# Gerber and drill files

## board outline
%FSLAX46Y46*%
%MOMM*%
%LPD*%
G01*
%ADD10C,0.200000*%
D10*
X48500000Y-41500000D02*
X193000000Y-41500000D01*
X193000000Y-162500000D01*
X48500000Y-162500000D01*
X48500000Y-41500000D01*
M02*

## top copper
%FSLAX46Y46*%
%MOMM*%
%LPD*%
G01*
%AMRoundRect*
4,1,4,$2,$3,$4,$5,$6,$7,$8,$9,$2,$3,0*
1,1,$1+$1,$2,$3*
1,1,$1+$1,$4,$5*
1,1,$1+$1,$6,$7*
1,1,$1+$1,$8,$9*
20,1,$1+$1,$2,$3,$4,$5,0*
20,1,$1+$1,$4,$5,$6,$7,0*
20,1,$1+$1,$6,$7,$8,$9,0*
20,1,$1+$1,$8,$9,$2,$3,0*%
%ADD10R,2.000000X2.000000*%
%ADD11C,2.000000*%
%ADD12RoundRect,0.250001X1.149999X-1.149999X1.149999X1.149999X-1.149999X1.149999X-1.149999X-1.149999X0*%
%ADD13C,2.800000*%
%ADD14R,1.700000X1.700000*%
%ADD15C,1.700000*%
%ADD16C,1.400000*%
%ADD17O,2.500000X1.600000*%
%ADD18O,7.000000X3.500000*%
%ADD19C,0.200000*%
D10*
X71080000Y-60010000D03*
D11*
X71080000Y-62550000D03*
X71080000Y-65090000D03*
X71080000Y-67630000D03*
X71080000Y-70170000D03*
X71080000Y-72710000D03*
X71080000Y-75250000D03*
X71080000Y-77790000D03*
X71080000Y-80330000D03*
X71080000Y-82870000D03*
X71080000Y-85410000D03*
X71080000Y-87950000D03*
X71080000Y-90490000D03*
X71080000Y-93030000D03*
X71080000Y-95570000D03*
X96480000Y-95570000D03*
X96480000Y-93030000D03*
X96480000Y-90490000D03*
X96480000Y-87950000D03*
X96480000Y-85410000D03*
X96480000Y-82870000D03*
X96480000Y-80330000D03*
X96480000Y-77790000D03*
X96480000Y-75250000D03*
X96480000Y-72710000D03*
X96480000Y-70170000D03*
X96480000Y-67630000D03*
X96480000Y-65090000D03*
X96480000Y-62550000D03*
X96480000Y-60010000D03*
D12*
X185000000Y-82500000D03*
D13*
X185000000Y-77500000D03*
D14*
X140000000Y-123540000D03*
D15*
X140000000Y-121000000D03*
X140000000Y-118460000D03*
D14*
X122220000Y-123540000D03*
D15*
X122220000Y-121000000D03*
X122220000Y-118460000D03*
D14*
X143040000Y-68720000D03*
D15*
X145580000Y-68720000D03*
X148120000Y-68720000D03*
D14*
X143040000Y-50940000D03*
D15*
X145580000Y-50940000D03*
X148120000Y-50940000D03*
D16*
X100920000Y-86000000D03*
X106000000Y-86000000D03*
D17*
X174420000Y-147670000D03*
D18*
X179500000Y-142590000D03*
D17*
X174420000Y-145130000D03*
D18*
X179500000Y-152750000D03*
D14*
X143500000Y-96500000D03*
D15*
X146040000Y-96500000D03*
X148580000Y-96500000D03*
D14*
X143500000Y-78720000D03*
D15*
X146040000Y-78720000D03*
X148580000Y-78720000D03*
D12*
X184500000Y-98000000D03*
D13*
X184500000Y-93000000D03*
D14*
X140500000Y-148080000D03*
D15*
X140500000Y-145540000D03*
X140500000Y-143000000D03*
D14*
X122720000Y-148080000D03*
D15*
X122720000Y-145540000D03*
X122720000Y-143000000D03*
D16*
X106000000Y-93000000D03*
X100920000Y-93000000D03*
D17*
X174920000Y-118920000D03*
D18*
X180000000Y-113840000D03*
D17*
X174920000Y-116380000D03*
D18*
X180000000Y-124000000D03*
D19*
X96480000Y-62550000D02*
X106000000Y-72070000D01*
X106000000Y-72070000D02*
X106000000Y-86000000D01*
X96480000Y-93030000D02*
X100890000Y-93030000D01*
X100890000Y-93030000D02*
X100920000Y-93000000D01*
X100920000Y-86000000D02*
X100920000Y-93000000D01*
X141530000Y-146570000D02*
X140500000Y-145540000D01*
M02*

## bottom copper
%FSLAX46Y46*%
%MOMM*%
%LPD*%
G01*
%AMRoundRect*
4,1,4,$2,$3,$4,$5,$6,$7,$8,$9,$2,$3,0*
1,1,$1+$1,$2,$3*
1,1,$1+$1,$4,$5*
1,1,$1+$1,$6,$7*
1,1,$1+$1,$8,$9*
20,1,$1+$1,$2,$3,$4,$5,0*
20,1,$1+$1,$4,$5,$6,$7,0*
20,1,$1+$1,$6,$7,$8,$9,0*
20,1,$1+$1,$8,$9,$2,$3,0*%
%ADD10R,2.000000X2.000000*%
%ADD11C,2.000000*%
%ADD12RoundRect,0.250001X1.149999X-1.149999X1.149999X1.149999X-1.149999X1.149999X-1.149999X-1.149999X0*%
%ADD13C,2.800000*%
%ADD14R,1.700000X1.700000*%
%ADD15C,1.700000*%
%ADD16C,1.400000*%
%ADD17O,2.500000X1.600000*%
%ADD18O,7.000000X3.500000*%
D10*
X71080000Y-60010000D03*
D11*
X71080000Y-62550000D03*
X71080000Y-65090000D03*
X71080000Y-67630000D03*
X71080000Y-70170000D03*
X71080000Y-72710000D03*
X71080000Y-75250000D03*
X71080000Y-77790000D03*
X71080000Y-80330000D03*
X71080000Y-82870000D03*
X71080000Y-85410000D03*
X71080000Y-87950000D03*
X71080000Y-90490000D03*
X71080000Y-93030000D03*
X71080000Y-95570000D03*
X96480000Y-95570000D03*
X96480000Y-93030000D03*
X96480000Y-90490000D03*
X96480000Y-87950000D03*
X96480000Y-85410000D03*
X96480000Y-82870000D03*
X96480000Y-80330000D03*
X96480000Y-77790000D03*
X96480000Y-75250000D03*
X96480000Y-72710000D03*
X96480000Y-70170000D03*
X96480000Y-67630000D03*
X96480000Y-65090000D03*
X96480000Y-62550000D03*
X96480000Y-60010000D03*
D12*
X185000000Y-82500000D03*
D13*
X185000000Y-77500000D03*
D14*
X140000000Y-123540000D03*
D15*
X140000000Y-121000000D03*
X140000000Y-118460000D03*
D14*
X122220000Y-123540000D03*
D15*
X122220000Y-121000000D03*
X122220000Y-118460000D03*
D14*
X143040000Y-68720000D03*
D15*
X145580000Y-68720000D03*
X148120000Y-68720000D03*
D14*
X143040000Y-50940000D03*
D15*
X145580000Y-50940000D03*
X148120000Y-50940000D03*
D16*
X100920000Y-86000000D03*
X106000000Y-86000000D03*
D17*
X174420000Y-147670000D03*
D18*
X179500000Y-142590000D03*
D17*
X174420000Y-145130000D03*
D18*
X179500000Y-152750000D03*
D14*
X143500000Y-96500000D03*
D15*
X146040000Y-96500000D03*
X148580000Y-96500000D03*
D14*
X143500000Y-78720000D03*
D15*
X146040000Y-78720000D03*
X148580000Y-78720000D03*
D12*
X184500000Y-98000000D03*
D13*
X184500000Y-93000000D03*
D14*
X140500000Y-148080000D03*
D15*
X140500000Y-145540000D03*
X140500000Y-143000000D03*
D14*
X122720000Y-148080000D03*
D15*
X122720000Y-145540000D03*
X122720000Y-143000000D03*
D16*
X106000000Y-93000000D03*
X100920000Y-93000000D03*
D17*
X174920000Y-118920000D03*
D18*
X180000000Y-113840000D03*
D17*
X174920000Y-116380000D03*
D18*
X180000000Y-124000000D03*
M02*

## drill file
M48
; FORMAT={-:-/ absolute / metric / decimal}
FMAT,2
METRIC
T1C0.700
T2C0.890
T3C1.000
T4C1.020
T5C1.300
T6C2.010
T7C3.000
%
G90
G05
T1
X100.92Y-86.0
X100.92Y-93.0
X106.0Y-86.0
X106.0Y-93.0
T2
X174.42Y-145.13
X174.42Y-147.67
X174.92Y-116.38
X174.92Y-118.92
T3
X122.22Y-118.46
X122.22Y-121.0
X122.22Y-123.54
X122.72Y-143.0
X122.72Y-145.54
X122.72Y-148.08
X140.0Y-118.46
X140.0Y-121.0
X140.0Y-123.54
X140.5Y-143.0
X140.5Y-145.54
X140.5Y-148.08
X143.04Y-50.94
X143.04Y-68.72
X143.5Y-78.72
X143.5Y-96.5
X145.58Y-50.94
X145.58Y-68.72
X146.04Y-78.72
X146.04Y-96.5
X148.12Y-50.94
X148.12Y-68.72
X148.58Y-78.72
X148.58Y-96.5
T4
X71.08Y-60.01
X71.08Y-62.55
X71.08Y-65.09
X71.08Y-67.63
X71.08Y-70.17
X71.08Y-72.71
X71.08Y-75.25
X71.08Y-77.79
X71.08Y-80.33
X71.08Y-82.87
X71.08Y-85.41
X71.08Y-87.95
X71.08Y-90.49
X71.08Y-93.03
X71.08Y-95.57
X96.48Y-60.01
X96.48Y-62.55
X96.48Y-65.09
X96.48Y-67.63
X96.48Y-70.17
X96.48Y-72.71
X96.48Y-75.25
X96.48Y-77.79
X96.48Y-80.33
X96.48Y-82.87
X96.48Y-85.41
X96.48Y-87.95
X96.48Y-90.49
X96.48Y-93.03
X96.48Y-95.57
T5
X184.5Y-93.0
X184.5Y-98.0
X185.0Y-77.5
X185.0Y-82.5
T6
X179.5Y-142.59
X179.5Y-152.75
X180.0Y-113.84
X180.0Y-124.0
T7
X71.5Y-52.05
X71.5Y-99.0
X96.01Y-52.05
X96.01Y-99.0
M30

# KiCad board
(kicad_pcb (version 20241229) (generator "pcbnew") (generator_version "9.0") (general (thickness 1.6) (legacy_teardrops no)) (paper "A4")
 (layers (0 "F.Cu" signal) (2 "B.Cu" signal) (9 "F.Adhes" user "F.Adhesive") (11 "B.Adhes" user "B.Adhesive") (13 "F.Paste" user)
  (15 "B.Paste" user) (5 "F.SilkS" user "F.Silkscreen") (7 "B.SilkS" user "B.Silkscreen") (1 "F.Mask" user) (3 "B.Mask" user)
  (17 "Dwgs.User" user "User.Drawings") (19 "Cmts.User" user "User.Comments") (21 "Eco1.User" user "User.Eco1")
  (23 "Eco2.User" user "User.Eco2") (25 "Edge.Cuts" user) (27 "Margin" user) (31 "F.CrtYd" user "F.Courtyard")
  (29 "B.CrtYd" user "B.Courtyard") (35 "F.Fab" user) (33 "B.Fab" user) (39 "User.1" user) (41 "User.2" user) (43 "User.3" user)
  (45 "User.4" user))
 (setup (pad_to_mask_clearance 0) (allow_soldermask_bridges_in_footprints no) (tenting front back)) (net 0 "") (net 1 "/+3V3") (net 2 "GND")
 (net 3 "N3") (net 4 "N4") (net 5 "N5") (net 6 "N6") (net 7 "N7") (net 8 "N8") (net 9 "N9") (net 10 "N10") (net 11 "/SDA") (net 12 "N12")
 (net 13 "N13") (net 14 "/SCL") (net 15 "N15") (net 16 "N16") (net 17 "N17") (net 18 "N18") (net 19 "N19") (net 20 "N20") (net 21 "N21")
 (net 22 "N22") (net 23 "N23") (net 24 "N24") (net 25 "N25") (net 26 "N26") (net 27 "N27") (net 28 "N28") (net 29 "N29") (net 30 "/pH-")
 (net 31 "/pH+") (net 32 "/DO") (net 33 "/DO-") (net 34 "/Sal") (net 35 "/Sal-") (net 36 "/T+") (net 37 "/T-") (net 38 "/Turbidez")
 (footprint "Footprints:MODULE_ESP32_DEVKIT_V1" (layer "F.Cu") (at 83.78 75.525)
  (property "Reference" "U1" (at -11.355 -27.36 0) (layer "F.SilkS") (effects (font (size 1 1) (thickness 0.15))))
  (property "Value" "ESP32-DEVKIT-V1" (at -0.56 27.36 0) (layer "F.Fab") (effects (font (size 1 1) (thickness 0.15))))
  (pad "" np_thru_hole circle (at -12.28 -23.475) (size 3 3) (drill 3) (layers "*.Cu" "*.Mask"))
  (pad "" np_thru_hole circle (at -12.28 23.475) (size 3 3) (drill 3) (layers "*.Cu" "*.Mask"))
  (pad "" np_thru_hole circle (at 12.23 -23.475) (size 3 3) (drill 3) (layers "*.Cu" "*.Mask"))
  (pad "" np_thru_hole circle (at 12.23 23.475) (size 3 3) (drill 3) (layers "*.Cu" "*.Mask"))
  (pad "1" thru_hole rect (at -12.7 -15.515) (size 2 2) (drill 1.02) (layers "*.Cu" "*.Mask") (remove_unused_layers no) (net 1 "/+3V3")
   (solder_mask_margin 0.102))
  (pad "2" thru_hole circle (at -12.7 -12.975) (size 2 2) (drill 1.02) (layers "*.Cu" "*.Mask") (remove_unused_layers no) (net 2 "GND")
   (solder_mask_margin 0.102))
  (pad "3" thru_hole circle (at -12.7 -10.435) (size 2 2) (drill 1.02) (layers "*.Cu" "*.Mask") (remove_unused_layers no) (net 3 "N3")
   (solder_mask_margin 0.102))
  (pad "4" thru_hole circle (at -12.7 -7.895) (size 2 2) (drill 1.02) (layers "*.Cu" "*.Mask") (remove_unused_layers no) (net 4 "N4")
   (solder_mask_margin 0.102))
  (pad "5" thru_hole circle (at -12.7 -5.355) (size 2 2) (drill 1.02) (layers "*.Cu" "*.Mask") (remove_unused_layers no) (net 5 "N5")
   (solder_mask_margin 0.102))
  (pad "6" thru_hole circle (at -12.7 -2.815) (size 2 2) (drill 1.02) (layers "*.Cu" "*.Mask") (remove_unused_layers no) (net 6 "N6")
   (solder_mask_margin 0.102))
  (pad "7" thru_hole circle (at -12.7 -0.275) (size 2 2) (drill 1.02) (layers "*.Cu" "*.Mask") (remove_unused_layers no) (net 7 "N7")
   (solder_mask_margin 0.102))
  (pad "8" thru_hole circle (at -12.7 2.265) (size 2 2) (drill 1.02) (layers "*.Cu" "*.Mask") (remove_unused_layers no) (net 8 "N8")
   (solder_mask_margin 0.102))
  (pad "9" thru_hole circle (at -12.7 4.805) (size 2 2) (drill 1.02) (layers "*.Cu" "*.Mask") (remove_unused_layers no) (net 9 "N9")
   (solder_mask_margin 0.102))
  (pad "10" thru_hole circle (at -12.7 7.345) (size 2 2) (drill 1.02) (layers "*.Cu" "*.Mask") (remove_unused_layers no) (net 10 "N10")
   (solder_mask_margin 0.102))
  (pad "11" thru_hole circle (at -12.7 9.885) (size 2 2) (drill 1.02) (layers "*.Cu" "*.Mask") (remove_unused_layers no) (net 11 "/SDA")
   (solder_mask_margin 0.102))
  (pad "12" thru_hole circle (at -12.7 12.425) (size 2 2) (drill 1.02) (layers "*.Cu" "*.Mask") (remove_unused_layers no) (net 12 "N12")
   (solder_mask_margin 0.102))
  (pad "13" thru_hole circle (at -12.7 14.965) (size 2 2) (drill 1.02) (layers "*.Cu" "*.Mask") (remove_unused_layers no) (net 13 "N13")
   (solder_mask_margin 0.102))
  (pad "14" thru_hole circle (at -12.7 17.505) (size 2 2) (drill 1.02) (layers "*.Cu" "*.Mask") (remove_unused_layers no) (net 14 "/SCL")
   (solder_mask_margin 0.102))
  (pad "15" thru_hole circle (at -12.7 20.045) (size 2 2) (drill 1.02) (layers "*.Cu" "*.Mask") (remove_unused_layers no) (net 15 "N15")
   (solder_mask_margin 0.102))
  (pad "16" thru_hole circle (at 12.7 20.045) (size 2 2) (drill 1.02) (layers "*.Cu" "*.Mask") (remove_unused_layers no) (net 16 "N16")
   (solder_mask_margin 0.102))
  (pad "17" thru_hole circle (at 12.7 17.505) (size 2 2) (drill 1.02) (layers "*.Cu" "*.Mask") (remove_unused_layers no) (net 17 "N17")
   (solder_mask_margin 0.102))
  (pad "18" thru_hole circle (at 12.7 14.965) (size 2 2) (drill 1.02) (layers "*.Cu" "*.Mask") (remove_unused_layers no) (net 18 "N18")
   (solder_mask_margin 0.102))
  (pad "19" thru_hole circle (at 12.7 12.425) (size 2 2) (drill 1.02) (layers "*.Cu" "*.Mask") (remove_unused_layers no) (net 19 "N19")
   (solder_mask_margin 0.102))
  (pad "20" thru_hole circle (at 12.7 9.885) (size 2 2) (drill 1.02) (layers "*.Cu" "*.Mask") (remove_unused_layers no) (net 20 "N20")
   (solder_mask_margin 0.102))
  (pad "21" thru_hole circle (at 12.7 7.345) (size 2 2) (drill 1.02) (layers "*.Cu" "*.Mask") (remove_unused_layers no) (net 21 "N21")
   (solder_mask_margin 0.102))
  (pad "22" thru_hole circle (at 12.7 4.805) (size 2 2) (drill 1.02) (layers "*.Cu" "*.Mask") (remove_unused_layers no) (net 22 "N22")
   (solder_mask_margin 0.102))
  (pad "23" thru_hole circle (at 12.7 2.265) (size 2 2) (drill 1.02) (layers "*.Cu" "*.Mask") (remove_unused_layers no) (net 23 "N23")
   (solder_mask_margin 0.102))
  (pad "24" thru_hole circle (at 12.7 -0.275) (size 2 2) (drill 1.02) (layers "*.Cu" "*.Mask") (remove_unused_layers no) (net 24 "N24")
   (solder_mask_margin 0.102))
  (pad "25" thru_hole circle (at 12.7 -2.815) (size 2 2) (drill 1.02) (layers "*.Cu" "*.Mask") (remove_unused_layers no) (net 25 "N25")
   (solder_mask_margin 0.102))
  (pad "26" thru_hole circle (at 12.7 -5.355) (size 2 2) (drill 1.02) (layers "*.Cu" "*.Mask") (remove_unused_layers no) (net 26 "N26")
   (solder_mask_margin 0.102))
  (pad "27" thru_hole circle (at 12.7 -7.895) (size 2 2) (drill 1.02) (layers "*.Cu" "*.Mask") (remove_unused_layers no) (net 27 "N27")
   (solder_mask_margin 0.102))
  (pad "28" thru_hole circle (at 12.7 -10.435) (size 2 2) (drill 1.02) (layers "*.Cu" "*.Mask") (remove_unused_layers no) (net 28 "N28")
   (solder_mask_margin 0.102))
  (pad "29" thru_hole circle (at 12.7 -12.975) (size 2 2) (drill 1.02) (layers "*.Cu" "*.Mask") (remove_unused_layers no) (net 2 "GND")
   (solder_mask_margin 0.102))
  (pad "30" thru_hole circle (at 12.7 -15.515) (size 2 2) (drill 1.02) (layers "*.Cu" "*.Mask") (remove_unused_layers no) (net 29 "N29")
   (solder_mask_margin 0.102))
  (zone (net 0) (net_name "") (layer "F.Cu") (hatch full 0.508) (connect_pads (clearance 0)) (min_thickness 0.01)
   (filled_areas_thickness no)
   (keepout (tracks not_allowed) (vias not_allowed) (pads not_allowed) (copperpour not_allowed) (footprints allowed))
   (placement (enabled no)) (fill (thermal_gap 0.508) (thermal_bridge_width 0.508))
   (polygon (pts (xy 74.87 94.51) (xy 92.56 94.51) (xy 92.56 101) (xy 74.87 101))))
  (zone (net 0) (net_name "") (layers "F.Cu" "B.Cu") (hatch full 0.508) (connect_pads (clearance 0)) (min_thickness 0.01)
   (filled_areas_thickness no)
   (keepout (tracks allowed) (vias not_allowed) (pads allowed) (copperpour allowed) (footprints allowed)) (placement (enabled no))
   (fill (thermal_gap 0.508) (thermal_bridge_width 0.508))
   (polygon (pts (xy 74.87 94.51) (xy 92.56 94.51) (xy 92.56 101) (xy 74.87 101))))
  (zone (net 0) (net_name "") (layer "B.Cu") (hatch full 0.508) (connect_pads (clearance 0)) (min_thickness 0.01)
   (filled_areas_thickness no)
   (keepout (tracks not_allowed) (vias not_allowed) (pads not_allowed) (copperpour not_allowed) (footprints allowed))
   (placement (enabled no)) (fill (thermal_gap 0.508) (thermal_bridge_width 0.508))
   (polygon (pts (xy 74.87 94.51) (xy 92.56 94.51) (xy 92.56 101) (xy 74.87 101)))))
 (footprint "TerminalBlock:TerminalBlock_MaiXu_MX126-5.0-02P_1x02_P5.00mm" (layer "F.Cu") (at 185 82.5 90)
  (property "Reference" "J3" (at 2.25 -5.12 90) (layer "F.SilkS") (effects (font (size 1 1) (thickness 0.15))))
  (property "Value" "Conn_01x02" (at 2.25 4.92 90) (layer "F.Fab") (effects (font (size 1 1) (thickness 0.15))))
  (pad "1" thru_hole roundrect (at 0 0 90) (size 2.8 2.8) (drill 1.3) (layers "*.Cu" "*.Mask") (remove_unused_layers no)
   (roundrect_rratio 0.089286) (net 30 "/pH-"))
  (pad "2" thru_hole circle (at 5 0 90) (size 2.8 2.8) (drill 1.3) (layers "*.Cu" "*.Mask") (remove_unused_layers no) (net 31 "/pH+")))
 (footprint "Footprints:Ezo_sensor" (layer "F.Cu") (at 119 114.46 90)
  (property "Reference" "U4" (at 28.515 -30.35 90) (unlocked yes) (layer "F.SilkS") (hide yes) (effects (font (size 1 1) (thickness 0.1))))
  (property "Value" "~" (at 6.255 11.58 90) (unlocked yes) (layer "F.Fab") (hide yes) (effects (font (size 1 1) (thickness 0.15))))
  (pad "1" thru_hole rect (at -9.08 21 180) (size 1.7 1.7) (drill 1) (layers "*.Cu" "*.Mask") (remove_unused_layers no) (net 1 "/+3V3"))
  (pad "2" thru_hole circle (at -6.54 21 180) (size 1.7 1.7) (drill 1) (layers "*.Cu" "*.Mask") (remove_unused_layers no) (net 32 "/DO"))
  (pad "3" thru_hole circle (at -4 21 180) (size 1.7 1.7) (drill 1) (layers "*.Cu" "*.Mask") (remove_unused_layers no) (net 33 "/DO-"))
  (pad "4" thru_hole rect (at -9.08 3.22 180) (size 1.7 1.7) (drill 1) (layers "*.Cu" "*.Mask") (remove_unused_layers no) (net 2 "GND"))
  (pad "5" thru_hole circle (at -6.54 3.22 180) (size 1.7 1.7) (drill 1) (layers "*.Cu" "*.Mask") (remove_unused_layers no) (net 11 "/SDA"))
  (pad "6" thru_hole circle (at -4 3.22 180) (size 1.7 1.7) (drill 1) (layers "*.Cu" "*.Mask") (remove_unused_layers no) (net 14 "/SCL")))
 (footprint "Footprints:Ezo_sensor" (layer "F.Cu") (at 112.875 90.8)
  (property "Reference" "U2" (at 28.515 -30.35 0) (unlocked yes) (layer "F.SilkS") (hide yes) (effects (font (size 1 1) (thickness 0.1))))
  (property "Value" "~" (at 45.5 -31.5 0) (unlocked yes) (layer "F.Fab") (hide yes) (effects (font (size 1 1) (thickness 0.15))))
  (pad "1" thru_hole rect (at 30.165 -22.08 90) (size 1.7 1.7) (drill 1) (layers "*.Cu" "*.Mask") (remove_unused_layers no) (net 1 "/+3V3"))
  (pad "2" thru_hole circle (at 32.705 -22.08 90) (size 1.7 1.7) (drill 1) (layers "*.Cu" "*.Mask") (remove_unused_layers no)
   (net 31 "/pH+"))
  (pad "3" thru_hole circle (at 35.245 -22.08 90) (size 1.7 1.7) (drill 1) (layers "*.Cu" "*.Mask") (remove_unused_layers no)
   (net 30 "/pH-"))
  (pad "4" thru_hole rect (at 30.165 -39.86 90) (size 1.7 1.7) (drill 1) (layers "*.Cu" "*.Mask") (remove_unused_layers no) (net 2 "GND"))
  (pad "5" thru_hole circle (at 32.705 -39.86 90) (size 1.7 1.7) (drill 1) (layers "*.Cu" "*.Mask") (remove_unused_layers no)
   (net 11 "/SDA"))
  (pad "6" thru_hole circle (at 35.245 -39.86 90) (size 1.7 1.7) (drill 1) (layers "*.Cu" "*.Mask") (remove_unused_layers no)
   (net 14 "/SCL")))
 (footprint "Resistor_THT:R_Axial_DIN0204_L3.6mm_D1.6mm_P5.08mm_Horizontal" (layer "F.Cu") (at 100.92 86)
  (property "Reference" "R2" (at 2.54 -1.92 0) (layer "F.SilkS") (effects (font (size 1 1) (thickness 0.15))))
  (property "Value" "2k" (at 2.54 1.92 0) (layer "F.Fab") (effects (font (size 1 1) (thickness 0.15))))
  (pad "1" thru_hole circle (at 0 0) (size 1.4 1.4) (drill 0.7) (layers "*.Cu" "*.Mask") (remove_unused_layers no) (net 17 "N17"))
  (pad "2" thru_hole circle (at 5.08 0) (size 1.4 1.4) (drill 0.7) (layers "*.Cu" "*.Mask") (remove_unused_layers no) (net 2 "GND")))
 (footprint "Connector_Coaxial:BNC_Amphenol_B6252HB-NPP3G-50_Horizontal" (layer "F.Cu") (at 174.42 147.67 -90)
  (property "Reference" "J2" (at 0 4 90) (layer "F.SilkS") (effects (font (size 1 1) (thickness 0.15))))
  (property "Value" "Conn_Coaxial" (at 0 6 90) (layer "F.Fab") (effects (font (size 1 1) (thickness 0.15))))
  (pad "1" thru_hole oval (at 0 0 270) (size 1.6 2.5) (drill 0.89) (layers "*.Cu" "*.Mask") (remove_unused_layers no) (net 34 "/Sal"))
  (pad "2" thru_hole oval (at -5.08 -5.08 270) (size 3.5 7) (drill 2.01) (layers "*.Cu" "*.Mask") (remove_unused_layers no) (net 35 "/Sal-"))
  (pad "2" thru_hole oval (at -2.54 0 270) (size 1.6 2.5) (drill 0.89) (layers "*.Cu" "*.Mask") (remove_unused_layers no) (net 35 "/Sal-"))
  (pad "2" thru_hole oval (at 5.08 -5.08 270) (size 3.5 7) (drill 2.01) (layers "*.Cu" "*.Mask") (remove_unused_layers no) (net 35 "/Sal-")))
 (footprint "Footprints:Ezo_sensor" (layer "F.Cu") (at 113.335 118.58)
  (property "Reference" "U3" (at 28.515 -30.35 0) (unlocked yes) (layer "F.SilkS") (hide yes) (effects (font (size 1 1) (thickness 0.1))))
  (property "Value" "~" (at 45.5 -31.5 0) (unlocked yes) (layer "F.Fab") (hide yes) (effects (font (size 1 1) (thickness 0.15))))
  (pad "1" thru_hole rect (at 30.165 -22.08 90) (size 1.7 1.7) (drill 1) (layers "*.Cu" "*.Mask") (remove_unused_layers no) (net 1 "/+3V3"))
  (pad "2" thru_hole circle (at 32.705 -22.08 90) (size 1.7 1.7) (drill 1) (layers "*.Cu" "*.Mask") (remove_unused_layers no) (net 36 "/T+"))
  (pad "3" thru_hole circle (at 35.245 -22.08 90) (size 1.7 1.7) (drill 1) (layers "*.Cu" "*.Mask") (remove_unused_layers no) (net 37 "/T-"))
  (pad "4" thru_hole rect (at 30.165 -39.86 90) (size 1.7 1.7) (drill 1) (layers "*.Cu" "*.Mask") (remove_unused_layers no) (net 2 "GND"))
  (pad "5" thru_hole circle (at 32.705 -39.86 90) (size 1.7 1.7) (drill 1) (layers "*.Cu" "*.Mask") (remove_unused_layers no)
   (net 11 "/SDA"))
  (pad "6" thru_hole circle (at 35.245 -39.86 90) (size 1.7 1.7) (drill 1) (layers "*.Cu" "*.Mask") (remove_unused_layers no)
   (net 14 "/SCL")))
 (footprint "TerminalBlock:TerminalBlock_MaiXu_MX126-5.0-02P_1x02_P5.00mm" (layer "F.Cu") (at 184.5 98 90)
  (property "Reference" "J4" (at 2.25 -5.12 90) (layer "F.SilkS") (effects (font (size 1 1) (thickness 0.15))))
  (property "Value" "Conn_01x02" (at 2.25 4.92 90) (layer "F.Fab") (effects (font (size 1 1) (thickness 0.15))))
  (pad "1" thru_hole roundrect (at 0 0 90) (size 2.8 2.8) (drill 1.3) (layers "*.Cu" "*.Mask") (remove_unused_layers no)
   (roundrect_rratio 0.089286) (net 37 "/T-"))
  (pad "2" thru_hole circle (at 5 0 90) (size 2.8 2.8) (drill 1.3) (layers "*.Cu" "*.Mask") (remove_unused_layers no) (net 36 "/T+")))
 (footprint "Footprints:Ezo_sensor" (layer "F.Cu") (at 119.5 139 90)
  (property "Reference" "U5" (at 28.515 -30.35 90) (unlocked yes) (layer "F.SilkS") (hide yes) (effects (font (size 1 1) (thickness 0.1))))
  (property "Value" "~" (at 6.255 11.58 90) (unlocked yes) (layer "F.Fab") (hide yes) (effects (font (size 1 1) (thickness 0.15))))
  (pad "1" thru_hole rect (at -9.08 21 180) (size 1.7 1.7) (drill 1) (layers "*.Cu" "*.Mask") (remove_unused_layers no) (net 1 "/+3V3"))
  (pad "2" thru_hole circle (at -6.54 21 180) (size 1.7 1.7) (drill 1) (layers "*.Cu" "*.Mask") (remove_unused_layers no) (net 34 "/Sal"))
  (pad "3" thru_hole circle (at -4 21 180) (size 1.7 1.7) (drill 1) (layers "*.Cu" "*.Mask") (remove_unused_layers no) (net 35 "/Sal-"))
  (pad "4" thru_hole rect (at -9.08 3.22 180) (size 1.7 1.7) (drill 1) (layers "*.Cu" "*.Mask") (remove_unused_layers no) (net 2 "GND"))
  (pad "5" thru_hole circle (at -6.54 3.22 180) (size 1.7 1.7) (drill 1) (layers "*.Cu" "*.Mask") (remove_unused_layers no) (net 11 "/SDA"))
  (pad "6" thru_hole circle (at -4 3.22 180) (size 1.7 1.7) (drill 1) (layers "*.Cu" "*.Mask") (remove_unused_layers no) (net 14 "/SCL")))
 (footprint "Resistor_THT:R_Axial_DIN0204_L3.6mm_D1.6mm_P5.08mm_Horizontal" (layer "F.Cu") (at 106 93 180)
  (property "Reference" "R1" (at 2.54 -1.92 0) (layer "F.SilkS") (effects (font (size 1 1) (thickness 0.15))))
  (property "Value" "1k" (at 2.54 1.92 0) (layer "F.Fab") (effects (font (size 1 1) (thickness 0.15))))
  (pad "1" thru_hole circle (at 0 0 180) (size 1.4 1.4) (drill 0.7) (layers "*.Cu" "*.Mask") (remove_unused_layers no) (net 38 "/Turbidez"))
  (pad "2" thru_hole circle (at 5.08 0 180) (size 1.4 1.4) (drill 0.7) (layers "*.Cu" "*.Mask") (remove_unused_layers no) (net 17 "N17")))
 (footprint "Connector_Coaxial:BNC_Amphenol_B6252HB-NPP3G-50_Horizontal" (layer "F.Cu") (at 174.92 118.92 -90)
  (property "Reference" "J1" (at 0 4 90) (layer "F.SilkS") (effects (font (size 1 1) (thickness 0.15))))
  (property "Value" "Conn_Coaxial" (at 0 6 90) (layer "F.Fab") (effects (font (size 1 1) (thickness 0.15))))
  (pad "1" thru_hole oval (at 0 0 270) (size 1.6 2.5) (drill 0.89) (layers "*.Cu" "*.Mask") (remove_unused_layers no) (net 32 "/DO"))
  (pad "2" thru_hole oval (at -5.08 -5.08 270) (size 3.5 7) (drill 2.01) (layers "*.Cu" "*.Mask") (remove_unused_layers no) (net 33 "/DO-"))
  (pad "2" thru_hole oval (at -2.54 0 270) (size 1.6 2.5) (drill 0.89) (layers "*.Cu" "*.Mask") (remove_unused_layers no) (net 33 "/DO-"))
  (pad "2" thru_hole oval (at 5.08 -5.08 270) (size 3.5 7) (drill 2.01) (layers "*.Cu" "*.Mask") (remove_unused_layers no) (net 33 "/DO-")))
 (gr_rect (start 48.5 41.5) (end 193 162.5) (stroke (width 0.2) (type solid)) (fill no) (layer "Edge.Cuts"))
 (segment (start 96.48 62.55) (end 106 72.07) (width 0.2) (layer "F.Cu") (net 2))
 (segment (start 106 72.07) (end 106 86) (width 0.2) (layer "F.Cu") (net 2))
 (segment (start 96.48 93.03) (end 100.89 93.03) (width 0.2) (layer "F.Cu") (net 17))
 (segment (start 100.89 93.03) (end 100.92 93) (width 0.2) (layer "F.Cu") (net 17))
 (segment (start 100.92 86) (end 100.92 93) (width 0.2) (layer "F.Cu") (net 17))
 (segment (start 141.53 146.57) (end 140.5 145.54) (width 0.2) (layer "F.Cu") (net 34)))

